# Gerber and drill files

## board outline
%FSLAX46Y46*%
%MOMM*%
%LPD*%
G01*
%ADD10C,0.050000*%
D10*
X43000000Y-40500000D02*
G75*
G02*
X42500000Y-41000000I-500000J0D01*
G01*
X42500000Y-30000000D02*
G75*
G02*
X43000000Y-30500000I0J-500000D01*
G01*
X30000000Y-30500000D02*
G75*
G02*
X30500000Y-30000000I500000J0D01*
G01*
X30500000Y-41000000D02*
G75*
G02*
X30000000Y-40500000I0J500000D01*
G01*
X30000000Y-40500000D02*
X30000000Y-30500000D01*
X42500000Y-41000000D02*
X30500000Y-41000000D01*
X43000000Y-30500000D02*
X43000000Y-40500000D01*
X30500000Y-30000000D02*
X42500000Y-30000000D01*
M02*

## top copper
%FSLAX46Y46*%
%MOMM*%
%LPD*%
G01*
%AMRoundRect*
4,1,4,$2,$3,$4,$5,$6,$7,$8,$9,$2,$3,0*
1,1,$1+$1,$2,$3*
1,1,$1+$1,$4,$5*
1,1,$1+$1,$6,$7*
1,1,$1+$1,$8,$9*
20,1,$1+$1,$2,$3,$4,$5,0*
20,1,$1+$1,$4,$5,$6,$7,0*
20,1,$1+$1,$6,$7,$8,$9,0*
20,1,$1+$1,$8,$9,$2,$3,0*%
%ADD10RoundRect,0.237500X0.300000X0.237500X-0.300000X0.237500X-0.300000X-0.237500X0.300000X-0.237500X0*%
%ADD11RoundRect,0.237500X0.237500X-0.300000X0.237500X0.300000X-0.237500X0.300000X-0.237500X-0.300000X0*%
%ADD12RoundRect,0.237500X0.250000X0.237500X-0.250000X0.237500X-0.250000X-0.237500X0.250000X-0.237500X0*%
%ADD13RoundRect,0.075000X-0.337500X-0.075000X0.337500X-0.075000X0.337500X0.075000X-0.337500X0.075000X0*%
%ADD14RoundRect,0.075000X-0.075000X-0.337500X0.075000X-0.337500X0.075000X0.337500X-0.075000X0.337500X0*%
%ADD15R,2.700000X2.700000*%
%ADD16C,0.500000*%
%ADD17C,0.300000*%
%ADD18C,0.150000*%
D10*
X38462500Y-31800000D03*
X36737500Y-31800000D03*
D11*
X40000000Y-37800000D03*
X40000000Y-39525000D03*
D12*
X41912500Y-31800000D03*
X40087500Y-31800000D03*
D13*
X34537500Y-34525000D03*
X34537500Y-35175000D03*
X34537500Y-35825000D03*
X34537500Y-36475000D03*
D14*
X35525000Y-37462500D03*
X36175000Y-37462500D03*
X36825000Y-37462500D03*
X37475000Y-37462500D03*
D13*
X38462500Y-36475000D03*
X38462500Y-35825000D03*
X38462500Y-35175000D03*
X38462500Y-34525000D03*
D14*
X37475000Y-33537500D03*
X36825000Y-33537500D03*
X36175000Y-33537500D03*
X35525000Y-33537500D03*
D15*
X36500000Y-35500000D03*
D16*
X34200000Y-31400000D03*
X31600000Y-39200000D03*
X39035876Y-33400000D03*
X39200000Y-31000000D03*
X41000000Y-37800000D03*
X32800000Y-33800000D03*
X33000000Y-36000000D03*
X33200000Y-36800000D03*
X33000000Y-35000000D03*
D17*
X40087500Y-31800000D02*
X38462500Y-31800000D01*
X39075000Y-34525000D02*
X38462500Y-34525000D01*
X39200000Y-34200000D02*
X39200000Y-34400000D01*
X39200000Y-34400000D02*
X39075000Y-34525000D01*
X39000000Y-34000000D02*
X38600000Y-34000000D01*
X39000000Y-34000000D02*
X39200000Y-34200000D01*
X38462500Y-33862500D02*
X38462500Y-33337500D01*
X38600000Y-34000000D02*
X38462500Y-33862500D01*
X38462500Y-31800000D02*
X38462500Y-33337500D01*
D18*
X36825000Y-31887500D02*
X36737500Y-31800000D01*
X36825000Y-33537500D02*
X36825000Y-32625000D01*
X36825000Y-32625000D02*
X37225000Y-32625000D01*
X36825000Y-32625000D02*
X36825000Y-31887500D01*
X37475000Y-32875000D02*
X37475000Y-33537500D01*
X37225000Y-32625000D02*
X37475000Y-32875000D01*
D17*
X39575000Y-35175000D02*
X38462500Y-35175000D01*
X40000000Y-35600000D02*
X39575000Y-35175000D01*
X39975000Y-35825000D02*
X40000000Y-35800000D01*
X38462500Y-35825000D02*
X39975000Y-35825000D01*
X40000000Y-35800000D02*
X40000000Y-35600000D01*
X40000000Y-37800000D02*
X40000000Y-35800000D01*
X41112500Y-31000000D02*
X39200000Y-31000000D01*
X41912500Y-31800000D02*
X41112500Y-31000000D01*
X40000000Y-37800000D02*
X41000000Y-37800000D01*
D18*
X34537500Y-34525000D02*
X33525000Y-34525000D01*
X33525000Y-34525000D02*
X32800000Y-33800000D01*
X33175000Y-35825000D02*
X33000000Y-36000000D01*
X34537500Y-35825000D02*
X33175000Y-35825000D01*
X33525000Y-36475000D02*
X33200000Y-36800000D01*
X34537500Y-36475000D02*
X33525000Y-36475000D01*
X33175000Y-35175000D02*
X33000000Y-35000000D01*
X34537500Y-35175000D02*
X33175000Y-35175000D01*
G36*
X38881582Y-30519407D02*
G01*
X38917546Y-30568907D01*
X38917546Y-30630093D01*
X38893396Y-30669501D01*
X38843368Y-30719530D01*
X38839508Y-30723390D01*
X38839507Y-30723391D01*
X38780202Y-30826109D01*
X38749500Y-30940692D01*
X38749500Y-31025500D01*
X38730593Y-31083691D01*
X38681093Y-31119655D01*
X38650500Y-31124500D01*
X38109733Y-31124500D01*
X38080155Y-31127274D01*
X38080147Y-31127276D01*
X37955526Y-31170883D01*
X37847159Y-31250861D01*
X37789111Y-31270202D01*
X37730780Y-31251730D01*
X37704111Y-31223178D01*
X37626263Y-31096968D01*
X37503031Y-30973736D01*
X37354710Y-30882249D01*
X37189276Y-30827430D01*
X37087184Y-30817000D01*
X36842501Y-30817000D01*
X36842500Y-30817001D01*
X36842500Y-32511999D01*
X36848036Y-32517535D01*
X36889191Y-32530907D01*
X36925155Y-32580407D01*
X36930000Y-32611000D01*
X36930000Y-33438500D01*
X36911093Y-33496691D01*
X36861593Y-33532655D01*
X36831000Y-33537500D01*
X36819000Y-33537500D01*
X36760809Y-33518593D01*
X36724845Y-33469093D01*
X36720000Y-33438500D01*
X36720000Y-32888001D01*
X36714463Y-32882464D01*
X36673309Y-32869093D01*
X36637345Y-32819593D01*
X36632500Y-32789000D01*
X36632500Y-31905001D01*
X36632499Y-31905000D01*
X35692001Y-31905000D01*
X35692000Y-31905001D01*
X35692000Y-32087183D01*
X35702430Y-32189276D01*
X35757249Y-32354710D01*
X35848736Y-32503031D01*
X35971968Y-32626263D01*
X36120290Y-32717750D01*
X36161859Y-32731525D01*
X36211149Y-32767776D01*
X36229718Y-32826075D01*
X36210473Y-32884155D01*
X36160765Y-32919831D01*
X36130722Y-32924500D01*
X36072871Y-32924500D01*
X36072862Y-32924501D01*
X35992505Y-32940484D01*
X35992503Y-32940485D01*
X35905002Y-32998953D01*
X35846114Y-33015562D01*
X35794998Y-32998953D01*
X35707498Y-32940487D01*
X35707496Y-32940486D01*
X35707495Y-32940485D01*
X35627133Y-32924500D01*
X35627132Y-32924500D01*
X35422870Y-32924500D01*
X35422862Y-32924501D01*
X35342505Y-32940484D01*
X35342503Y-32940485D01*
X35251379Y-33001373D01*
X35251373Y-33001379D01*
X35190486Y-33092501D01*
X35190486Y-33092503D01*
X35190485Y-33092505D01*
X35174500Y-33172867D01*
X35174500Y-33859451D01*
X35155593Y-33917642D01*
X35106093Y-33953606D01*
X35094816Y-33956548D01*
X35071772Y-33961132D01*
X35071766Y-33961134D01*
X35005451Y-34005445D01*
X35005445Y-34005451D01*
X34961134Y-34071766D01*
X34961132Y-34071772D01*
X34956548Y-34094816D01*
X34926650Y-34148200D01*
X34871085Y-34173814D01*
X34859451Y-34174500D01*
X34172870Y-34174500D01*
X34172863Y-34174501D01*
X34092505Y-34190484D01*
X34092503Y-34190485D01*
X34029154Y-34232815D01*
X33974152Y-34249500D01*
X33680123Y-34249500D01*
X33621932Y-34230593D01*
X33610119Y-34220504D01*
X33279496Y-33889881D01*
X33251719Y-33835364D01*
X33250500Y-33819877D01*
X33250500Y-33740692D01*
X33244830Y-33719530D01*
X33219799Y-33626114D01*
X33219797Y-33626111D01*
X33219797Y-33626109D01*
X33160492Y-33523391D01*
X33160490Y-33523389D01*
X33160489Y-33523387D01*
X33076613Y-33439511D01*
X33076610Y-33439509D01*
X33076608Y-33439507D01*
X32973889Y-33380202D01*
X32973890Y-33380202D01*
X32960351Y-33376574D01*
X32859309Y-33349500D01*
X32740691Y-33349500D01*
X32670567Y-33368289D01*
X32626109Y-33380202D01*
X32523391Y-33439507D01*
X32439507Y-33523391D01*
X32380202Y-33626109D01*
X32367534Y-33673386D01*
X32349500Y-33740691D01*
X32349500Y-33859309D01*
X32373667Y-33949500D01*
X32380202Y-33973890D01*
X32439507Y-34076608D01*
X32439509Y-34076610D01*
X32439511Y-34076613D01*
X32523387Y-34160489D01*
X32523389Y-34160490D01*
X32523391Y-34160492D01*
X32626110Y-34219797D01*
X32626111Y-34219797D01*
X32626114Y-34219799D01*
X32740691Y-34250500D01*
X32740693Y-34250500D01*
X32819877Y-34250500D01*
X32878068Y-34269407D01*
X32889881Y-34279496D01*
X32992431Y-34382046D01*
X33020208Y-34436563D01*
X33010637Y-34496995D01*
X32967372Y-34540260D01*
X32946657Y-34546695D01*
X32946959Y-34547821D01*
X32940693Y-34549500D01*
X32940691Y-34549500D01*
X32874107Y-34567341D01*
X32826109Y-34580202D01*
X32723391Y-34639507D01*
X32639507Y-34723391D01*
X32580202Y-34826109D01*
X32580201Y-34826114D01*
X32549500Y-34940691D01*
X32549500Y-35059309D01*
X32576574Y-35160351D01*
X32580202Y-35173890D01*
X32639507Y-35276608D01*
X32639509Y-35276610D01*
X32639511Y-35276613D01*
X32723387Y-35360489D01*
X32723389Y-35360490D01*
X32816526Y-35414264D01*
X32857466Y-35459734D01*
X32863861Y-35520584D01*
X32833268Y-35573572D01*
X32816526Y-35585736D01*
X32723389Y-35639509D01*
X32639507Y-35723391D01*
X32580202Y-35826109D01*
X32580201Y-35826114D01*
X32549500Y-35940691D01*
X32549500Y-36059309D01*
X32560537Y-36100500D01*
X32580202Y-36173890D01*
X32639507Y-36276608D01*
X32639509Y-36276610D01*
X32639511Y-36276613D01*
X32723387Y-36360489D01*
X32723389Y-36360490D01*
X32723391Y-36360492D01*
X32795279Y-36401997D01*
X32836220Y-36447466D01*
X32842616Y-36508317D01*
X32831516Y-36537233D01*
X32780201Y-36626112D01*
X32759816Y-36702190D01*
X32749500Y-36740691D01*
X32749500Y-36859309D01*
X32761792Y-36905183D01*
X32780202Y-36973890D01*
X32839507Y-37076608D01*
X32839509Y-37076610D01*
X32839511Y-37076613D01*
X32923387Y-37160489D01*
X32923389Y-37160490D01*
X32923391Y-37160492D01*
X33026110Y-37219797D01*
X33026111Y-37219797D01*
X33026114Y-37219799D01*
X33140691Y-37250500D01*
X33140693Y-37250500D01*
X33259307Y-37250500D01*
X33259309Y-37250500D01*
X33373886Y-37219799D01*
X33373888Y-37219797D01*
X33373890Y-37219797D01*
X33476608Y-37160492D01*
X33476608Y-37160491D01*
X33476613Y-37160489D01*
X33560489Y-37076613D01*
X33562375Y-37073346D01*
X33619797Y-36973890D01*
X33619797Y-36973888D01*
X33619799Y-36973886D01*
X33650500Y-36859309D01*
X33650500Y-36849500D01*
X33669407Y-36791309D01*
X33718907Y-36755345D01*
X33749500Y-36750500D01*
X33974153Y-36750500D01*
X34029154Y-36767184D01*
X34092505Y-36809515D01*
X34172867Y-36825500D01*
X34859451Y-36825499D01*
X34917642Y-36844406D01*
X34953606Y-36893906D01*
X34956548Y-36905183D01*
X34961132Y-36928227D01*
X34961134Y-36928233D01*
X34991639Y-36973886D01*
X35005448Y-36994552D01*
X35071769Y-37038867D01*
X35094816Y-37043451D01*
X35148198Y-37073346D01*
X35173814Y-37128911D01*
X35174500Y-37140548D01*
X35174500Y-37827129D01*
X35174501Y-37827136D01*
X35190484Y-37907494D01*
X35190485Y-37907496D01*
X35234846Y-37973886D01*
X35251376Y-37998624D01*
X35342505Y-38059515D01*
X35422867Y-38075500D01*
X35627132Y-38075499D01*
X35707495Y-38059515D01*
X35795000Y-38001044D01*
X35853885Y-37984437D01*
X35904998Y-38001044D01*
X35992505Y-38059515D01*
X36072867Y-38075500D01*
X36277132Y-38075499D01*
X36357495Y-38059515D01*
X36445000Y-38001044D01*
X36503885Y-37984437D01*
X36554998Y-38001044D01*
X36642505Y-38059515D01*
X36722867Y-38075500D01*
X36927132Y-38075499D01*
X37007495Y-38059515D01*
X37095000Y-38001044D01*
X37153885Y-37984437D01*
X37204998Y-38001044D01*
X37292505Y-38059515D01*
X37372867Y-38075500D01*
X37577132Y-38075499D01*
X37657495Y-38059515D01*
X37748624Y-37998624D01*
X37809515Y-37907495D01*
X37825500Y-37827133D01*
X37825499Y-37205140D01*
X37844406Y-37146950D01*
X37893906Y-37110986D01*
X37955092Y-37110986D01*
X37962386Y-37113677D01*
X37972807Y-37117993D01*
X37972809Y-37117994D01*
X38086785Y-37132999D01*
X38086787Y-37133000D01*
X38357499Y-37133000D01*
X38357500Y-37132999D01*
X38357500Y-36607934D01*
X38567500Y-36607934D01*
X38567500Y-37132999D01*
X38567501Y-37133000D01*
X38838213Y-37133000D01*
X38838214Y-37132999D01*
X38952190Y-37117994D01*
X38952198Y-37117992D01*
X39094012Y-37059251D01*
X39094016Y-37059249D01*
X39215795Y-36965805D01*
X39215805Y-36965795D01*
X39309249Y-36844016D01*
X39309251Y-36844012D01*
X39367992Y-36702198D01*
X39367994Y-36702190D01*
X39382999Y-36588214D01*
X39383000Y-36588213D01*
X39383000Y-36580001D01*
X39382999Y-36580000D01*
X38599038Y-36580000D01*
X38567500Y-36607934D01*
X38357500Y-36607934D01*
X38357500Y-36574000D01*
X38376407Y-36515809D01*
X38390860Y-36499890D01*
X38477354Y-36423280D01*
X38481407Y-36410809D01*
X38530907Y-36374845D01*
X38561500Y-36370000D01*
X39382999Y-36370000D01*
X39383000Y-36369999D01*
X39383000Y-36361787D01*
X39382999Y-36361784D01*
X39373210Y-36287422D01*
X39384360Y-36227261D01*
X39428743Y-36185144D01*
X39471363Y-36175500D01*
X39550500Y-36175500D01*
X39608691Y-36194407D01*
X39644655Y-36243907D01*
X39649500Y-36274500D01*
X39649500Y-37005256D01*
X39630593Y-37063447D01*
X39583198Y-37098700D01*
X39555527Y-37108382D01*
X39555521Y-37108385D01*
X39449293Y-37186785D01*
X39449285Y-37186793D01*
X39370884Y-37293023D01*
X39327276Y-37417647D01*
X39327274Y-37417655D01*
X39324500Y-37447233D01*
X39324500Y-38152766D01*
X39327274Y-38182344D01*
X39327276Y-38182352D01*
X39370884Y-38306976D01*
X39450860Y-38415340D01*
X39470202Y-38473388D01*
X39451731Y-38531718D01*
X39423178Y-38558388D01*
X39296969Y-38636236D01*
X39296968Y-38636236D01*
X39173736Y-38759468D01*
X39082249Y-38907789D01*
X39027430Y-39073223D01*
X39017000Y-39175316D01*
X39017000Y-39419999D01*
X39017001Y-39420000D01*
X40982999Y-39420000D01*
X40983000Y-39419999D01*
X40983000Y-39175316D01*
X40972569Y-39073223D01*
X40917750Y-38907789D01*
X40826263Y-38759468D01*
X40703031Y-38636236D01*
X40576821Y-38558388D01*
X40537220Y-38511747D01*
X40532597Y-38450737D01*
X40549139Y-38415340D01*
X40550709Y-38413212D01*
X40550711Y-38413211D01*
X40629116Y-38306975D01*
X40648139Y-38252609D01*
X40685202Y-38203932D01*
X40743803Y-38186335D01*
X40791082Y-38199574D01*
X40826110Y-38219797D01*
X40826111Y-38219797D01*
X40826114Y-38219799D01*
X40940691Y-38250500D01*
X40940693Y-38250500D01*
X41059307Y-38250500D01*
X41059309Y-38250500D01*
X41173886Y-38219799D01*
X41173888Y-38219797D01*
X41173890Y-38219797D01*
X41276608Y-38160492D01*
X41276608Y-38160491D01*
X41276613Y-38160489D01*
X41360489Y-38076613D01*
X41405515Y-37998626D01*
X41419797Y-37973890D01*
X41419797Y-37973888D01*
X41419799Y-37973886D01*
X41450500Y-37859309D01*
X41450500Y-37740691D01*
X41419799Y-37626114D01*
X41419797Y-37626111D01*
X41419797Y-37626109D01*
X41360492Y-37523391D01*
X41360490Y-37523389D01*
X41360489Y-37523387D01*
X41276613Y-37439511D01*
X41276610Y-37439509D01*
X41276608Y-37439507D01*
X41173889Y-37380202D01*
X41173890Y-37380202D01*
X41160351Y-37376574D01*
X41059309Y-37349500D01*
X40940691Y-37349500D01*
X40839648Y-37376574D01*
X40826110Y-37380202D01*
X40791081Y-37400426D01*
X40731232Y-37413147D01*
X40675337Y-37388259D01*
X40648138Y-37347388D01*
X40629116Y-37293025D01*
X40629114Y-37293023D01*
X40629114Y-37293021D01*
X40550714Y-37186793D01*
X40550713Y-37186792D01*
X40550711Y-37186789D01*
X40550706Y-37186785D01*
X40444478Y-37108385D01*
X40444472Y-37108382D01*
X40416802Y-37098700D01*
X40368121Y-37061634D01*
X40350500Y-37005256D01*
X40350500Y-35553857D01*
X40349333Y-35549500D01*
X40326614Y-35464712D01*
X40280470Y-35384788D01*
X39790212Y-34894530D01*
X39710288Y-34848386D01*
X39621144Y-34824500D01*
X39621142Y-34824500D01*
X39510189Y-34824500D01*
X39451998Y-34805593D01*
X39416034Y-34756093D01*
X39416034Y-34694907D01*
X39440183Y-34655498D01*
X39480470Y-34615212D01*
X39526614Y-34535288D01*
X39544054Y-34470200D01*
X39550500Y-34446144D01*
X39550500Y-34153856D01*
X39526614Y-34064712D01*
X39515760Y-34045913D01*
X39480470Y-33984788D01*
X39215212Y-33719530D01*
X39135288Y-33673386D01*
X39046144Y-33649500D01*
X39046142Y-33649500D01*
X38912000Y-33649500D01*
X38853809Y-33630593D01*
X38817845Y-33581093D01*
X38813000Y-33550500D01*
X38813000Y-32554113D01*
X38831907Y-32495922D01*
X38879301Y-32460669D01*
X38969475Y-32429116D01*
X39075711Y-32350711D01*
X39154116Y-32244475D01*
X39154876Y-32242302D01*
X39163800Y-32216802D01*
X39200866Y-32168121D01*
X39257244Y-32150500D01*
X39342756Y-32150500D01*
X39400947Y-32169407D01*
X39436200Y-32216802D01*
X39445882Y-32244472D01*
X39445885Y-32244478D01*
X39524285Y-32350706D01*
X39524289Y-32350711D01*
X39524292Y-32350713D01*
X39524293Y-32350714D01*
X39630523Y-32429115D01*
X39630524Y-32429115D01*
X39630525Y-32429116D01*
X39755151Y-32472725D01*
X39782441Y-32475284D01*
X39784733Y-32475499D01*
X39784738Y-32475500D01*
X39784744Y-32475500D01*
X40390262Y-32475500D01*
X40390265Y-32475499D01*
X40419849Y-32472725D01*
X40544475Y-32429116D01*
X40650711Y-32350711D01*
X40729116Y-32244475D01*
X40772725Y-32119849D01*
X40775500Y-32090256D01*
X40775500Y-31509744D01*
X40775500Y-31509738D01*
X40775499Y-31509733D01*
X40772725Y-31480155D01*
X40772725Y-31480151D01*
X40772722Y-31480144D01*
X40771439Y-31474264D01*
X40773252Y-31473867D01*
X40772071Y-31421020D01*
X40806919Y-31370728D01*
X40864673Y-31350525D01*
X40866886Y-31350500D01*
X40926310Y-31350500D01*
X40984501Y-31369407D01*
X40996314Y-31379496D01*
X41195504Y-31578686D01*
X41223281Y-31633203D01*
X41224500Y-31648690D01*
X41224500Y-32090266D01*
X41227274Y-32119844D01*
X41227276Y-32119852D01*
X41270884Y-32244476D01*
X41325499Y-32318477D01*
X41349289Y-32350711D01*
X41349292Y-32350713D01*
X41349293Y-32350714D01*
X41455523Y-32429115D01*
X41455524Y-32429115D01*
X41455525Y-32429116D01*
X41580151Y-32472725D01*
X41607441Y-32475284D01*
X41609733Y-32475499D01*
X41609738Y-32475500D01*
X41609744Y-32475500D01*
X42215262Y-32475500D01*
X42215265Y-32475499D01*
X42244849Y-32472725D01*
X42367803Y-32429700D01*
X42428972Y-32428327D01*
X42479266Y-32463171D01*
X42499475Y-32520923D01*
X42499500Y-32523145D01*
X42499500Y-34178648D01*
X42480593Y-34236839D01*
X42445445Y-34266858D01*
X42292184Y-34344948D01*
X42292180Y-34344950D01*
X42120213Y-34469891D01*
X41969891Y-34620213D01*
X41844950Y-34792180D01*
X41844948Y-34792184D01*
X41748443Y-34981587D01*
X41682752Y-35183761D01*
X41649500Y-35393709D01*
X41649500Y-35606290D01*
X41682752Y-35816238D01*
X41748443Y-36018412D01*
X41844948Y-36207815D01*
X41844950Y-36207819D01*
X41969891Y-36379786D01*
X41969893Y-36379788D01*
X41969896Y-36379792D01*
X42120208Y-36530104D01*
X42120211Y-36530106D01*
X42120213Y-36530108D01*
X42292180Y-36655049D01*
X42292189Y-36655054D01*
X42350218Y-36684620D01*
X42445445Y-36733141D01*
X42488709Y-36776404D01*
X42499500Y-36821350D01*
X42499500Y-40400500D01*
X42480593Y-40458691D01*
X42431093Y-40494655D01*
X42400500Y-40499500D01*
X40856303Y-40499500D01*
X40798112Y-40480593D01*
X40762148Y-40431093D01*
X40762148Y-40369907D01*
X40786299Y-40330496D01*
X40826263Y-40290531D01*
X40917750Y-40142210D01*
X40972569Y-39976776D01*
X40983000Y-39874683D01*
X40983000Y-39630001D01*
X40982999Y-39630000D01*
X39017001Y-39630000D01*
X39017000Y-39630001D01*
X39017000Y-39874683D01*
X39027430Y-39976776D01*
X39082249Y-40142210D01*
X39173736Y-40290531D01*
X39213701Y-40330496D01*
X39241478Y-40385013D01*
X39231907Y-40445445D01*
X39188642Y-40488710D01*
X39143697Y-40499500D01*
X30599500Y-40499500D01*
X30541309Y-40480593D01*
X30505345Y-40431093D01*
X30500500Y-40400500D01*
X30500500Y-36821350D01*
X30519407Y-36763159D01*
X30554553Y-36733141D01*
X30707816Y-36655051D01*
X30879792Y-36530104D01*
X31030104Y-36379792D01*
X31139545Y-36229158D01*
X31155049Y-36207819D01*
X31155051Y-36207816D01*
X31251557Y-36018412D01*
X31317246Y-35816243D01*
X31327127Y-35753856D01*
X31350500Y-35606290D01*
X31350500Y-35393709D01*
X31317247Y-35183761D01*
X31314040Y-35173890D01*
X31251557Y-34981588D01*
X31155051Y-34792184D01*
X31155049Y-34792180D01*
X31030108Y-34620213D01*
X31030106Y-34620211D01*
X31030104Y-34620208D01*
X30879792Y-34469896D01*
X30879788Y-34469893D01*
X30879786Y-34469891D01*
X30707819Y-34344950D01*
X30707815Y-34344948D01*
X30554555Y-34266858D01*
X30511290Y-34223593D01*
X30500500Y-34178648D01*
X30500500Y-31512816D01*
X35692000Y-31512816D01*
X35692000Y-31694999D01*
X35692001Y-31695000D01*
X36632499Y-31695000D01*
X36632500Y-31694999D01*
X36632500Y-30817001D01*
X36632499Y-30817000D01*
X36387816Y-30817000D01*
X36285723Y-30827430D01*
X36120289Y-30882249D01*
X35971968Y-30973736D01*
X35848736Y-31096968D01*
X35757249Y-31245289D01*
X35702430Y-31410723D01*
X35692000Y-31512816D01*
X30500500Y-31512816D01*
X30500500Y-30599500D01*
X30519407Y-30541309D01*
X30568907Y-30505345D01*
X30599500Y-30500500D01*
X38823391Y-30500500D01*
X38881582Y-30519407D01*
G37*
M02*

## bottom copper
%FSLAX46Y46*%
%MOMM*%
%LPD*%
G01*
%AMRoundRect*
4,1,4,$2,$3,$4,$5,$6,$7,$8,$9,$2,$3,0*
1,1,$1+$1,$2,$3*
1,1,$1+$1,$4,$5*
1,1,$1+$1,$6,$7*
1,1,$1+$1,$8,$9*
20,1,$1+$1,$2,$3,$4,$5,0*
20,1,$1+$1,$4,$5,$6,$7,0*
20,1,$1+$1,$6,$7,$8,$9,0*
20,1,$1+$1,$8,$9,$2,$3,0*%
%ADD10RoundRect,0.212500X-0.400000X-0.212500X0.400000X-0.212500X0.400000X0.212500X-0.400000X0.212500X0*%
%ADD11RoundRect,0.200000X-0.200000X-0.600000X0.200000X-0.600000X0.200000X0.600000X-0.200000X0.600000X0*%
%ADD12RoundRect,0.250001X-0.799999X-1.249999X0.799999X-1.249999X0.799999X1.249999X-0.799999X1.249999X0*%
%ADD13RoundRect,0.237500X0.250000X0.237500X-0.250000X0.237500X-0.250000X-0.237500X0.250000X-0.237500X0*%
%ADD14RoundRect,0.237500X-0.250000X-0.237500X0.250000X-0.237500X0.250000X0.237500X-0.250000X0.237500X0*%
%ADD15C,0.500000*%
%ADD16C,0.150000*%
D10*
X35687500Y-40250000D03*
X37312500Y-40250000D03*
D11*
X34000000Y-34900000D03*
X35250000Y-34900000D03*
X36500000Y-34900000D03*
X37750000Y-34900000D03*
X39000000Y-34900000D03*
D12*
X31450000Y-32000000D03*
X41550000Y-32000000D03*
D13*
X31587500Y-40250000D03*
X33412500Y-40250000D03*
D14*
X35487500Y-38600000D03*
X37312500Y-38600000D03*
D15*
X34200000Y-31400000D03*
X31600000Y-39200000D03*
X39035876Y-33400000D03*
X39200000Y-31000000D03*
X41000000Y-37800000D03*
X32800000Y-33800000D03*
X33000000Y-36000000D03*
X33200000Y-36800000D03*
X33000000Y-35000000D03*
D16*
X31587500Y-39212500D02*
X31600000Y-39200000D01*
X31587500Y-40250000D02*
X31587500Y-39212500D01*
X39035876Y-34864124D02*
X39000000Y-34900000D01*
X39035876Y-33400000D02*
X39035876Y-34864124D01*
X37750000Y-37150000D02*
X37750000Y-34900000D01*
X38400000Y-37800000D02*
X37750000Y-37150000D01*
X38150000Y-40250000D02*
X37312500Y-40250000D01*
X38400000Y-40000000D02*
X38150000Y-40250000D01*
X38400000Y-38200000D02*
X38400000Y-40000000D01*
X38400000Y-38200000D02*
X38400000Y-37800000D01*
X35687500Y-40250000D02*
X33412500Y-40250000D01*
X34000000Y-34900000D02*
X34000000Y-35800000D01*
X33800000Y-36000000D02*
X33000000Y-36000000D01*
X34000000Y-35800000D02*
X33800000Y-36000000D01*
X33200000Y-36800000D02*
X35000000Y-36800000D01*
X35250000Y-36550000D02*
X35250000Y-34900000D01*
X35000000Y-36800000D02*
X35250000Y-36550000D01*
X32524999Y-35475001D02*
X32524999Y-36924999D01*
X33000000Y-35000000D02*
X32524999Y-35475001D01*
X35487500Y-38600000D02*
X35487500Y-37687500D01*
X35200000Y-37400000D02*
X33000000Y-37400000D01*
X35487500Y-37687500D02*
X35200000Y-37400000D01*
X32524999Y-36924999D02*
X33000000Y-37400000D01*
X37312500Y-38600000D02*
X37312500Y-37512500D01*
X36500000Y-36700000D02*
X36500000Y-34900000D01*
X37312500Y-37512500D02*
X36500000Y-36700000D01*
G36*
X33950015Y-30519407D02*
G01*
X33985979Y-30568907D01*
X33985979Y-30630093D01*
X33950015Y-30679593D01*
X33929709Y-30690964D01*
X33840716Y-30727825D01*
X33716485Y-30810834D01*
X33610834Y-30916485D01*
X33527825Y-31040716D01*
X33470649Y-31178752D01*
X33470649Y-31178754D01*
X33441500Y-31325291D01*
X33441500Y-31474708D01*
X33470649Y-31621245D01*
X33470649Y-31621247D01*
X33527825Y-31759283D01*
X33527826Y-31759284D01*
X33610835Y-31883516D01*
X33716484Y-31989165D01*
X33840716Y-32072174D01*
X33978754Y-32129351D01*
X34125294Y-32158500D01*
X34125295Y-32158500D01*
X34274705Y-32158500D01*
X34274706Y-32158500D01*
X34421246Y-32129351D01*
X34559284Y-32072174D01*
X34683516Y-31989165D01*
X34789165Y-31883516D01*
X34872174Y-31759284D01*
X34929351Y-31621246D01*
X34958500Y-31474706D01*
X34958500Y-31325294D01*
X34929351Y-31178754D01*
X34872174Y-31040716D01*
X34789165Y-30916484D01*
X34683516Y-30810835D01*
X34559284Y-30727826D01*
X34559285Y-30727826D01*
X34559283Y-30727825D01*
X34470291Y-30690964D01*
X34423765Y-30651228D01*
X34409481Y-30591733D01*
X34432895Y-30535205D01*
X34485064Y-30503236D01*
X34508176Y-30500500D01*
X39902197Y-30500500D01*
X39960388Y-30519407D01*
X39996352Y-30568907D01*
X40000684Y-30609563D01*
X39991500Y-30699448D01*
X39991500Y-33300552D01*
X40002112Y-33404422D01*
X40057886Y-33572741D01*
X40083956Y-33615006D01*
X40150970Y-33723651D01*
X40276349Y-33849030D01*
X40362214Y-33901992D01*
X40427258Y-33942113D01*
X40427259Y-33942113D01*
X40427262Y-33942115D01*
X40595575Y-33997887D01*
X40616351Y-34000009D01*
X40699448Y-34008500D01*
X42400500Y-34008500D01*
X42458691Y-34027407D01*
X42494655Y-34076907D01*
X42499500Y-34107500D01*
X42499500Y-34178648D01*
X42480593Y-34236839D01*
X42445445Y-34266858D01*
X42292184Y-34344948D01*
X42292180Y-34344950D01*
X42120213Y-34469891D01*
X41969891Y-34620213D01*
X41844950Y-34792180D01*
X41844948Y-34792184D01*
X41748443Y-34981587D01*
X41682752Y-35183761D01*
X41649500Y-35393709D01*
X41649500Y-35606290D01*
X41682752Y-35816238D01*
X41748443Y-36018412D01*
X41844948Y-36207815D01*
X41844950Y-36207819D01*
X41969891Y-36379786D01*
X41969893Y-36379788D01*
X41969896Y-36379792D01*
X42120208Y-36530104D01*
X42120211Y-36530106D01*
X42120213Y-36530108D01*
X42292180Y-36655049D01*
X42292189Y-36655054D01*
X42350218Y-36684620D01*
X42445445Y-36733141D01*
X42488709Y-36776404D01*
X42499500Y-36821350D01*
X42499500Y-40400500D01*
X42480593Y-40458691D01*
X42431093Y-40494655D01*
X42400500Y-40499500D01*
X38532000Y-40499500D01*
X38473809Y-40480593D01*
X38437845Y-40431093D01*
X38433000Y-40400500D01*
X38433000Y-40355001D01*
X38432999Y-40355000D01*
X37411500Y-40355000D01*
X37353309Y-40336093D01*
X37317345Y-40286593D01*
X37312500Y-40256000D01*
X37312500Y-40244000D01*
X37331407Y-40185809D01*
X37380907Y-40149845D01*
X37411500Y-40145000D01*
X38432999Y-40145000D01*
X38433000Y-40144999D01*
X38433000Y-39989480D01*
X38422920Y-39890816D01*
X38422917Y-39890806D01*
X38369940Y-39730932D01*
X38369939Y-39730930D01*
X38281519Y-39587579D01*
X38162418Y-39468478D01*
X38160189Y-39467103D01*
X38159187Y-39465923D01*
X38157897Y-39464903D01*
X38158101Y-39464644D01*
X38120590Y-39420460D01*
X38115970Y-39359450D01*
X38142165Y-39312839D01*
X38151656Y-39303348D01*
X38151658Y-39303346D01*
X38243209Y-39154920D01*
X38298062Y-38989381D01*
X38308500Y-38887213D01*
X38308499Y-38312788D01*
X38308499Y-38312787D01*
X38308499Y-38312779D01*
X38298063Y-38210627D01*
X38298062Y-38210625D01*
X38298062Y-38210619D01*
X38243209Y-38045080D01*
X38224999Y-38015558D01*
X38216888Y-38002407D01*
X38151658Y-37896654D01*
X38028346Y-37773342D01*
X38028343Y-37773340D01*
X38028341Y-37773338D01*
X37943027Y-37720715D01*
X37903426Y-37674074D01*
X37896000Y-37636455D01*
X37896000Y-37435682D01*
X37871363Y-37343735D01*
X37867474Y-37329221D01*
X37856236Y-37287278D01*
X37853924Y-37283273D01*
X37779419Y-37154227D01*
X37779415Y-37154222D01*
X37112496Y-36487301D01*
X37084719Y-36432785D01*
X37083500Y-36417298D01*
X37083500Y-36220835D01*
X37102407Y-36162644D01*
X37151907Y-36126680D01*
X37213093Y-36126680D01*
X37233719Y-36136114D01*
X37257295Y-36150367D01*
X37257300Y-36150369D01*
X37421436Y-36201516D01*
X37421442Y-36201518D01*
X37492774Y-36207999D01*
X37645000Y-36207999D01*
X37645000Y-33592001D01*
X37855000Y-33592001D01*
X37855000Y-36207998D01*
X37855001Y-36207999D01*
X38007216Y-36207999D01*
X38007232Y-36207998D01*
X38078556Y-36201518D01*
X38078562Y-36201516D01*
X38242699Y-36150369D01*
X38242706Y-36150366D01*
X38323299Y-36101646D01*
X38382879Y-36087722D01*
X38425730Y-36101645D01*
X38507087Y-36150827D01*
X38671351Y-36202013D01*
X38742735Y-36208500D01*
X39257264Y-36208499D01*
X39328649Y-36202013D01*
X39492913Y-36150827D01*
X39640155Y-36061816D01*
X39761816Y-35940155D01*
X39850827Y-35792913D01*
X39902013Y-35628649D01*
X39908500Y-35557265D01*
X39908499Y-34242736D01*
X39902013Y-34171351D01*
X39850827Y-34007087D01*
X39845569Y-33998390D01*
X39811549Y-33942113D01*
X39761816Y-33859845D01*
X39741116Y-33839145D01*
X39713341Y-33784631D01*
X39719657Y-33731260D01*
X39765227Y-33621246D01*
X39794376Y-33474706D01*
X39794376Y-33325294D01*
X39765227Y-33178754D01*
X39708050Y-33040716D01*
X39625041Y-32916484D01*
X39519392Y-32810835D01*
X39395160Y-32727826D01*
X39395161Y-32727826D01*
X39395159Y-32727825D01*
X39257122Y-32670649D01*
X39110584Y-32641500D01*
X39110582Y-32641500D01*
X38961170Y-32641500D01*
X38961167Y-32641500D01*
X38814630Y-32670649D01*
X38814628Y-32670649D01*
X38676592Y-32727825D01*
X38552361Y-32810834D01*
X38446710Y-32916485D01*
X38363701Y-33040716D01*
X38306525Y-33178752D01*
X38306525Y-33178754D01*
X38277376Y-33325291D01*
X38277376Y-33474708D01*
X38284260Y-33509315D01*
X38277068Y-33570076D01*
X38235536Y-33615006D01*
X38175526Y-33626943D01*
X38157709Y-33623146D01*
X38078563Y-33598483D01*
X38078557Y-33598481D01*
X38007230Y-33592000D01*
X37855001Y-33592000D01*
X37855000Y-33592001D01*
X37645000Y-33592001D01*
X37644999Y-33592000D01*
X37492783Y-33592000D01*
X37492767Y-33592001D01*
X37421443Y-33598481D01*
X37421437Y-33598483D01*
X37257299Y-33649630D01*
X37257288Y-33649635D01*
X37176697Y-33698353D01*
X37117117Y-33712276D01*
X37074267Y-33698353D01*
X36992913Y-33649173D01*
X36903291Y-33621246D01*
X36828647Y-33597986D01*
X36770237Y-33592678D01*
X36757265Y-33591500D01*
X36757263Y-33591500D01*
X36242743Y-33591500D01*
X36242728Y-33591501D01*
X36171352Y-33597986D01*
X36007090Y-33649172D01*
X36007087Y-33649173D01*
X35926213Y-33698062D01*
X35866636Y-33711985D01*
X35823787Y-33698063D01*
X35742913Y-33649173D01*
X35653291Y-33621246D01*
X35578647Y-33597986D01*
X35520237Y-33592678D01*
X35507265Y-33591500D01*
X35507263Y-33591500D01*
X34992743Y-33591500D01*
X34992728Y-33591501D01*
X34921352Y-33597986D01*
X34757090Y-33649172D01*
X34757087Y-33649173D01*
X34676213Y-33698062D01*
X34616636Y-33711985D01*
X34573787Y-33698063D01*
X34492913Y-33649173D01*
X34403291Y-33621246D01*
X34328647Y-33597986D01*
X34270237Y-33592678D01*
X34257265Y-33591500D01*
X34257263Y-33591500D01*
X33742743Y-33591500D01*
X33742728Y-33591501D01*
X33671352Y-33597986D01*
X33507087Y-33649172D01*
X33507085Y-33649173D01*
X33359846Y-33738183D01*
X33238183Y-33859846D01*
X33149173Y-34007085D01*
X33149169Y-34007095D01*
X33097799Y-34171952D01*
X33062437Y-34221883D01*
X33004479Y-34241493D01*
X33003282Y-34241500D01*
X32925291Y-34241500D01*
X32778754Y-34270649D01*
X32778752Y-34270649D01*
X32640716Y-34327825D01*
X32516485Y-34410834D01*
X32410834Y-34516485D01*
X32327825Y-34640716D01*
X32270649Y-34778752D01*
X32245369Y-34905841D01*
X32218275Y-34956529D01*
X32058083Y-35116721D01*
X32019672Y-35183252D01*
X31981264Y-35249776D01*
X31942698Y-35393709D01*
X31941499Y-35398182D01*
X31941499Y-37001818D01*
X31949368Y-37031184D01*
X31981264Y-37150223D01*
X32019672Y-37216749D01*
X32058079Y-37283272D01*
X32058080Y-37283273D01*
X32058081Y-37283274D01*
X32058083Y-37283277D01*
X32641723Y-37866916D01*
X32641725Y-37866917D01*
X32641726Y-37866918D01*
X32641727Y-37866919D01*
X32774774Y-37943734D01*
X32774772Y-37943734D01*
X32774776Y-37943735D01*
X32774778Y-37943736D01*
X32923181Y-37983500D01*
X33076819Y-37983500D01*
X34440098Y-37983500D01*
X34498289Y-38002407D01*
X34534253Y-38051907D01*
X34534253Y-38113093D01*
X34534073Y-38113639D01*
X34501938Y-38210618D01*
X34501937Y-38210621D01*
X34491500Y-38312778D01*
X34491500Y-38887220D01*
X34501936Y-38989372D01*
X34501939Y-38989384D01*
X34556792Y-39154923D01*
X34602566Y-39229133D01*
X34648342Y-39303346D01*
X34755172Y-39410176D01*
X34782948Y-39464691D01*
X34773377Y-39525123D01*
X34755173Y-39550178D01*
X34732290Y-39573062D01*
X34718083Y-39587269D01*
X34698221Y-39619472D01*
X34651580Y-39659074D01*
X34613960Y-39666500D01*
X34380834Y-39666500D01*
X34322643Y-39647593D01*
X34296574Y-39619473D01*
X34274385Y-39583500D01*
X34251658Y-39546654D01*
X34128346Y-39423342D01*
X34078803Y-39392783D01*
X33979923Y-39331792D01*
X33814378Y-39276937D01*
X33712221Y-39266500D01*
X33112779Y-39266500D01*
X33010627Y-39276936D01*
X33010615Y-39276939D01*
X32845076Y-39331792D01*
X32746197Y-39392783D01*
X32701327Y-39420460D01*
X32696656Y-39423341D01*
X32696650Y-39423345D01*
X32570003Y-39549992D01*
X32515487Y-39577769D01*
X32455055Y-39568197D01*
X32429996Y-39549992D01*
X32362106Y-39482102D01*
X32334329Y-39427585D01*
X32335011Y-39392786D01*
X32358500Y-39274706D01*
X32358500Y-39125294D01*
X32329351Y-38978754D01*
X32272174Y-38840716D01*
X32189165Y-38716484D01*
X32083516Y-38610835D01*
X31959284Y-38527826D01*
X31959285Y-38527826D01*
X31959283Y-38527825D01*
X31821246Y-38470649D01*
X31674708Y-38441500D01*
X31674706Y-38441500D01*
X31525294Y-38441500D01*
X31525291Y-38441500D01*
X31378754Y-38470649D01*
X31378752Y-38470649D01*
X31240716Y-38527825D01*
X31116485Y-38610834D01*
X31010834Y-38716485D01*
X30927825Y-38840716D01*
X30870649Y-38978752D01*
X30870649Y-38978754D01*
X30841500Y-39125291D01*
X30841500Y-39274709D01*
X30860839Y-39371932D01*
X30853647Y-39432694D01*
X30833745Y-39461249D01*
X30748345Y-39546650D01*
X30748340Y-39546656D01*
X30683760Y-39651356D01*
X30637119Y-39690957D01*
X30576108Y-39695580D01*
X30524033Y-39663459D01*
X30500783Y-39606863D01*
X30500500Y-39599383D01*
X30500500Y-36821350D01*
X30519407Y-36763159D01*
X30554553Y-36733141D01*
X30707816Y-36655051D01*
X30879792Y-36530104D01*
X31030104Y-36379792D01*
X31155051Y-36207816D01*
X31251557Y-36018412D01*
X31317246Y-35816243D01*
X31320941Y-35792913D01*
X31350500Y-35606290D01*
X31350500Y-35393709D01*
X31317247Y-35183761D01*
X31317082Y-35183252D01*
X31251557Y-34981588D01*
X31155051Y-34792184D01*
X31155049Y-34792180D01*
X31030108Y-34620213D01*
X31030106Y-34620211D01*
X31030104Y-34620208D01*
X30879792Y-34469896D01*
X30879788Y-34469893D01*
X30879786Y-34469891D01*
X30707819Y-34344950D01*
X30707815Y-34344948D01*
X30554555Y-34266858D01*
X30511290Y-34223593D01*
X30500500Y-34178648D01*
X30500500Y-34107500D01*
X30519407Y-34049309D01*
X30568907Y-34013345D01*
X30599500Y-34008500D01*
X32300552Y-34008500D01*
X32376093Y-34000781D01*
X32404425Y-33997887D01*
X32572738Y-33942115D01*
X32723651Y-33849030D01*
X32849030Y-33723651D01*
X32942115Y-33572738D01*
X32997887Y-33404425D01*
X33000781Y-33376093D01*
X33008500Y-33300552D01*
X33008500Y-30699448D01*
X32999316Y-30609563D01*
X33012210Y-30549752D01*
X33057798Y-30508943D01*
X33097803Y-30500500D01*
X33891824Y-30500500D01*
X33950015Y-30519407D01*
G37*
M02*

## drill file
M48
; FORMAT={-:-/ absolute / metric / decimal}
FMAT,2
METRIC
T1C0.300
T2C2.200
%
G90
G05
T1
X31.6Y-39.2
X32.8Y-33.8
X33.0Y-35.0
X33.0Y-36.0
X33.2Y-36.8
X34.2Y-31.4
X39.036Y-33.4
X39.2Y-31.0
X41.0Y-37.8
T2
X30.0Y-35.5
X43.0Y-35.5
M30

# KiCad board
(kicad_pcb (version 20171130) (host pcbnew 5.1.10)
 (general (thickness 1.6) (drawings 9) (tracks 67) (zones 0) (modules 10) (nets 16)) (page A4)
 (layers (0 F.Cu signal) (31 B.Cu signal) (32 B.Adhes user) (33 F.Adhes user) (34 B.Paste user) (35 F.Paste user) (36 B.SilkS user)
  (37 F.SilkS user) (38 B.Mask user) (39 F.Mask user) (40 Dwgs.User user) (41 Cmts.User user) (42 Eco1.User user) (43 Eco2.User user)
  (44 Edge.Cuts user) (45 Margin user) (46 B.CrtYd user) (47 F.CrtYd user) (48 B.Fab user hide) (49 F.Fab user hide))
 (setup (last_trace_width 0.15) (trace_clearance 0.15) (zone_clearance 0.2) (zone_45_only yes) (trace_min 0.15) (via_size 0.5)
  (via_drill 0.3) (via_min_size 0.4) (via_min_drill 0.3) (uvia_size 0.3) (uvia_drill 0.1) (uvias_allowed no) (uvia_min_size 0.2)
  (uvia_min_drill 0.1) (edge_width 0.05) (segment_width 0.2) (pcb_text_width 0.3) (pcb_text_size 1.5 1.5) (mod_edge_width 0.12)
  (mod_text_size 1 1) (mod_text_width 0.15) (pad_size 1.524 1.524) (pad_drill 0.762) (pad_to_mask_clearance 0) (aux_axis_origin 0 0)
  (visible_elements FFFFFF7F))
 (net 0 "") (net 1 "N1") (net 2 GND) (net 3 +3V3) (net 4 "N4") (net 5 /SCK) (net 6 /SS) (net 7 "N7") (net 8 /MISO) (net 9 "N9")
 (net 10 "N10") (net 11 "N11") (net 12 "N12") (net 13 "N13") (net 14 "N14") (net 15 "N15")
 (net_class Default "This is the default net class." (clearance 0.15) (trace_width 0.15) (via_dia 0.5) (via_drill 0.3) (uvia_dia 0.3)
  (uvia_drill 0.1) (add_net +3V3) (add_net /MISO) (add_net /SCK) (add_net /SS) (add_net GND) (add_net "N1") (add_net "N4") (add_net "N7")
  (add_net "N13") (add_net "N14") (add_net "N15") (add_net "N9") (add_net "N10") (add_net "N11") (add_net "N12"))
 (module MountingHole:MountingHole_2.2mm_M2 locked (layer F.Cu) (at 43 35.5)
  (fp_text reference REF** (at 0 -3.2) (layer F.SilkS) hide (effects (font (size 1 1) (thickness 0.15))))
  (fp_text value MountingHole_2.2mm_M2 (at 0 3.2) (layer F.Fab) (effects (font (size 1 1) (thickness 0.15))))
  (pad 1 np_thru_hole circle (at 0 0) (size 2.2 2.2) (drill 2.2) (layers *.Cu *.Mask)))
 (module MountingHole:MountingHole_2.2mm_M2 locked (layer F.Cu) (at 30 35.5)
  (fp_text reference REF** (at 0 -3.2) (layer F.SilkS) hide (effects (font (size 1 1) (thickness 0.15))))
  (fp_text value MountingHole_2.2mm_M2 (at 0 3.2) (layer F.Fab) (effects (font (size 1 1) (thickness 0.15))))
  (pad 1 np_thru_hole circle (at 0 0) (size 2.2 2.2) (drill 2.2) (layers *.Cu *.Mask)))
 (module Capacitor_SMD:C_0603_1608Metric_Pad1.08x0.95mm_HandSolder (layer F.Cu) (at 37.6 31.8 180)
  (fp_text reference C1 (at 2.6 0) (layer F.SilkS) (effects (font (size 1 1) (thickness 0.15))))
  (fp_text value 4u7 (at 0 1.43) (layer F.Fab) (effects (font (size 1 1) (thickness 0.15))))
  (pad 1 smd roundrect (at -0.8625 0 180) (size 1.075 0.95) (layers F.Cu F.Paste F.Mask) (roundrect_rratio 0.25) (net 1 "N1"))
  (pad 2 smd roundrect (at 0.8625 0 180) (size 1.075 0.95) (layers F.Cu F.Paste F.Mask) (roundrect_rratio 0.25) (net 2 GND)))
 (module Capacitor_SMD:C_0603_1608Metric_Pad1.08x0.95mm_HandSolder (layer F.Cu) (at 40 38.6625 90)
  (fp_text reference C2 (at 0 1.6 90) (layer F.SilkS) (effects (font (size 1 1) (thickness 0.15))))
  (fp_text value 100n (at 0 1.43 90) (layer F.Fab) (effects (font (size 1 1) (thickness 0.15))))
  (pad 2 smd roundrect (at 0.8625 0 90) (size 1.075 0.95) (layers F.Cu F.Paste F.Mask) (roundrect_rratio 0.25) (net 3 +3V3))
  (pad 1 smd roundrect (at -0.8625 0 90) (size 1.075 0.95) (layers F.Cu F.Paste F.Mask) (roundrect_rratio 0.25) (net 2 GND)))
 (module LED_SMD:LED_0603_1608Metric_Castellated (layer B.Cu) (at 36.5 40.25)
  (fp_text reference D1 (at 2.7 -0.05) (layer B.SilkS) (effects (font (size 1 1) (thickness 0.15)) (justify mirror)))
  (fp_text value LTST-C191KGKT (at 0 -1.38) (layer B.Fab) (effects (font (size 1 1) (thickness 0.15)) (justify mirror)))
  (pad 1 smd roundrect (at -0.8125 0) (size 1.225 0.85) (layers B.Cu B.Paste B.Mask) (roundrect_rratio 0.25) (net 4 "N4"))
  (pad 2 smd roundrect (at 0.8125 0) (size 1.225 0.85) (layers B.Cu B.Paste B.Mask) (roundrect_rratio 0.25) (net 3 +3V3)))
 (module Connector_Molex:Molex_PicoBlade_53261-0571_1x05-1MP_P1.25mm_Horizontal (layer B.Cu) (at 36.5 32.5)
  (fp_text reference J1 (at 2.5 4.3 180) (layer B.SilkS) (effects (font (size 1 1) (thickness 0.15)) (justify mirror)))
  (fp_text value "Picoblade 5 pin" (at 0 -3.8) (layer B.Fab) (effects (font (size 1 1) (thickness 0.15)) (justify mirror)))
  (pad 1 smd roundrect (at -2.5 2.4) (size 0.8 1.6) (layers B.Cu B.Paste B.Mask) (roundrect_rratio 0.25) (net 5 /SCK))
  (pad 2 smd roundrect (at -1.25 2.4) (size 0.8 1.6) (layers B.Cu B.Paste B.Mask) (roundrect_rratio 0.25) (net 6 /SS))
  (pad 3 smd roundrect (at 0 2.4) (size 0.8 1.6) (layers B.Cu B.Paste B.Mask) (roundrect_rratio 0.25) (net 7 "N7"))
  (pad 4 smd roundrect (at 1.25 2.4) (size 0.8 1.6) (layers B.Cu B.Paste B.Mask) (roundrect_rratio 0.25) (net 3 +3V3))
  (pad 5 smd roundrect (at 2.5 2.4) (size 0.8 1.6) (layers B.Cu B.Paste B.Mask) (roundrect_rratio 0.25) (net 2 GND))
  (pad MP smd roundrect (at -5.05 -0.5) (size 2.1 3) (layers B.Cu B.Paste B.Mask) (roundrect_rratio 0.119048))
  (pad MP smd roundrect (at 5.05 -0.5) (size 2.1 3) (layers B.Cu B.Paste B.Mask) (roundrect_rratio 0.119048)))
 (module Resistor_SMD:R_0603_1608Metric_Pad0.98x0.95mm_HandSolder (layer F.Cu) (at 41 31.8 180)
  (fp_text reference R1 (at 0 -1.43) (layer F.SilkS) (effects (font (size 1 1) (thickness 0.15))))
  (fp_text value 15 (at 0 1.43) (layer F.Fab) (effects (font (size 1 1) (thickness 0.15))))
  (pad 1 smd roundrect (at -0.9125 0 180) (size 0.975 0.95) (layers F.Cu F.Paste F.Mask) (roundrect_rratio 0.25) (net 3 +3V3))
  (pad 2 smd roundrect (at 0.9125 0 180) (size 0.975 0.95) (layers F.Cu F.Paste F.Mask) (roundrect_rratio 0.25) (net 1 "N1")))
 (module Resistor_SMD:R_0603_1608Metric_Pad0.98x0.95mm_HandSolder (layer B.Cu) (at 32.5 40.25 180)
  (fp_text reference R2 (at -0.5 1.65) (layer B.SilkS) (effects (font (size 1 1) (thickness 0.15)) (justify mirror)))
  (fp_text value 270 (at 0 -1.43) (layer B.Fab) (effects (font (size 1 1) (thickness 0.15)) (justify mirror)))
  (pad 2 smd roundrect (at 0.9125 0 180) (size 0.975 0.95) (layers B.Cu B.Paste B.Mask) (roundrect_rratio 0.25) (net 2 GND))
  (pad 1 smd roundrect (at -0.9125 0 180) (size 0.975 0.95) (layers B.Cu B.Paste B.Mask) (roundrect_rratio 0.25) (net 4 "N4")))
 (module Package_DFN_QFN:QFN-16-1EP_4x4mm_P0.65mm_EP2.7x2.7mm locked (layer F.Cu) (at 36.5 35.5)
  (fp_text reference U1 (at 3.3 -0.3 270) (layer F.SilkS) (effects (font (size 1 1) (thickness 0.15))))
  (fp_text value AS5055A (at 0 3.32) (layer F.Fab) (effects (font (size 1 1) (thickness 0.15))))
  (pad 1 smd roundrect (at -1.9625 -0.975) (size 0.825 0.3) (layers F.Cu F.Paste F.Mask) (roundrect_rratio 0.25) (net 3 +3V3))
  (pad 2 smd roundrect (at -1.9625 -0.325) (size 0.825 0.3) (layers F.Cu F.Paste F.Mask) (roundrect_rratio 0.25) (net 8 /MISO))
  (pad 3 smd roundrect (at -1.9625 0.325) (size 0.825 0.3) (layers F.Cu F.Paste F.Mask) (roundrect_rratio 0.25) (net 5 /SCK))
  (pad 4 smd roundrect (at -1.9625 0.975) (size 0.825 0.3) (layers F.Cu F.Paste F.Mask) (roundrect_rratio 0.25) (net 6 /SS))
  (pad 5 smd roundrect (at -0.975 1.9625) (size 0.3 0.825) (layers F.Cu F.Paste F.Mask) (roundrect_rratio 0.25) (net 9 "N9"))
  (pad 6 smd roundrect (at -0.325 1.9625) (size 0.3 0.825) (layers F.Cu F.Paste F.Mask) (roundrect_rratio 0.25) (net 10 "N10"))
  (pad 7 smd roundrect (at 0.325 1.9625) (size 0.3 0.825) (layers F.Cu F.Paste F.Mask) (roundrect_rratio 0.25) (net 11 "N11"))
  (pad 8 smd roundrect (at 0.975 1.9625) (size 0.3 0.825) (layers F.Cu F.Paste F.Mask) (roundrect_rratio 0.25) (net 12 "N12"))
  (pad 9 smd roundrect (at 1.9625 0.975) (size 0.825 0.3) (layers F.Cu F.Paste F.Mask) (roundrect_rratio 0.25) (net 2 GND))
  (pad 10 smd roundrect (at 1.9625 0.325) (size 0.825 0.3) (layers F.Cu F.Paste F.Mask) (roundrect_rratio 0.25) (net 3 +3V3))
  (pad 11 smd roundrect (at 1.9625 -0.325) (size 0.825 0.3) (layers F.Cu F.Paste F.Mask) (roundrect_rratio 0.25) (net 3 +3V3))
  (pad 12 smd roundrect (at 1.9625 -0.975) (size 0.825 0.3) (layers F.Cu F.Paste F.Mask) (roundrect_rratio 0.25) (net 1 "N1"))
  (pad 13 smd roundrect (at 0.975 -1.9625) (size 0.3 0.825) (layers F.Cu F.Paste F.Mask) (roundrect_rratio 0.25) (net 2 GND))
  (pad 14 smd roundrect (at 0.325 -1.9625) (size 0.3 0.825) (layers F.Cu F.Paste F.Mask) (roundrect_rratio 0.25) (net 2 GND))
  (pad 15 smd roundrect (at -0.325 -1.9625) (size 0.3 0.825) (layers F.Cu F.Paste F.Mask) (roundrect_rratio 0.25) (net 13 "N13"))
  (pad 16 smd roundrect (at -0.975 -1.9625) (size 0.3 0.825) (layers F.Cu F.Paste F.Mask) (roundrect_rratio 0.25) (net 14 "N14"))
  (pad 17 smd rect (at 0 0) (size 2.7 2.7) (layers F.Cu F.Mask) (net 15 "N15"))
  (pad "" smd roundrect (at -0.675 -0.675) (size 1.09 1.09) (layers F.Paste) (roundrect_rratio 0.229358))
  (pad "" smd roundrect (at -0.675 0.675) (size 1.09 1.09) (layers F.Paste) (roundrect_rratio 0.229358))
  (pad "" smd roundrect (at 0.675 -0.675) (size 1.09 1.09) (layers F.Paste) (roundrect_rratio 0.229358))
  (pad "" smd roundrect (at 0.675 0.675) (size 1.09 1.09) (layers F.Paste) (roundrect_rratio 0.229358)))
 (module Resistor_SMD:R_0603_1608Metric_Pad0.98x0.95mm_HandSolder (layer B.Cu) (at 36.4 38.6)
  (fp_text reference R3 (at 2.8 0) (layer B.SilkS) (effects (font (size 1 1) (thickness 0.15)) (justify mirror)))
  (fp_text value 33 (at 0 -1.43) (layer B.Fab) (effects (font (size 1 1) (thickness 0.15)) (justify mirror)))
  (pad 1 smd roundrect (at -0.9125 0) (size 0.975 0.95) (layers B.Cu B.Paste B.Mask) (roundrect_rratio 0.25) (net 8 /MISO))
  (pad 2 smd roundrect (at 0.9125 0) (size 0.975 0.95) (layers B.Cu B.Paste B.Mask) (roundrect_rratio 0.25) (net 7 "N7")))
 (gr_arc (start 42.5 40.5) (end 42.5 41) (angle -90) (layer Edge.Cuts) (width 0.05))
 (gr_arc (start 42.5 30.5) (end 43 30.5) (angle -90) (layer Edge.Cuts) (width 0.05))
 (gr_arc (start 30.5 30.5) (end 30.5 30) (angle -90) (layer Edge.Cuts) (width 0.05))
 (gr_arc (start 30.5 40.5) (end 30 40.5) (angle -90) (layer Edge.Cuts) (width 0.05))
 (gr_line (start 30 40.5) (end 30 30.5) (layer Edge.Cuts) (width 0.05))
 (gr_line (start 42.5 41) (end 30.5 41) (layer Edge.Cuts) (width 0.05))
 (gr_line (start 43 30.5) (end 43 40.5) (layer Edge.Cuts) (width 0.05))
 (gr_line (start 30.5 30) (end 42.5 30) (layer Edge.Cuts) (width 0.05))
 (via (at 34.2 31.4) (size 0.5) (drill 0.3) (layers F.Cu B.Cu) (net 2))
 (segment (start 40.0875 31.8) (end 38.4625 31.8) (width 0.3) (layer F.Cu) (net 1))
 (segment (start 39.075 34.525) (end 38.4625 34.525) (width 0.3) (layer F.Cu) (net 1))
 (segment (start 39.2 34.2) (end 39.2 34.4) (width 0.3) (layer F.Cu) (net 1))
 (segment (start 39.2 34.4) (end 39.075 34.525) (width 0.3) (layer F.Cu) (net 1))
 (segment (start 39 34) (end 38.6 34) (width 0.3) (layer F.Cu) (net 1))
 (segment (start 39 34) (end 39.2 34.2) (width 0.3) (layer F.Cu) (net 1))
 (segment (start 38.4625 33.8625) (end 38.4625 33.3375) (width 0.3) (layer F.Cu) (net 1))
 (segment (start 38.6 34) (end 38.4625 33.8625) (width 0.3) (layer F.Cu) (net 1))
 (segment (start 38.4625 31.8) (end 38.4625 33.3375) (width 0.3) (layer F.Cu) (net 1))
 (segment (start 36.825 31.8875) (end 36.7375 31.8) (width 0.15) (layer F.Cu) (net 2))
 (segment (start 36.825 33.5375) (end 36.825 32.625) (width 0.15) (layer F.Cu) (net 2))
 (segment (start 36.825 32.625) (end 37.225 32.625) (width 0.15) (layer F.Cu) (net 2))
 (segment (start 36.825 32.625) (end 36.825 31.8875) (width 0.15) (layer F.Cu) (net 2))
 (segment (start 37.475 32.875) (end 37.475 33.5375) (width 0.15) (layer F.Cu) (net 2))
 (segment (start 37.225 32.625) (end 37.475 32.875) (width 0.15) (layer F.Cu) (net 2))
 (via (at 31.6 39.2) (size 0.5) (drill 0.3) (layers F.Cu B.Cu) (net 2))
 (segment (start 31.5875 39.2125) (end 31.6 39.2) (width 0.15) (layer B.Cu) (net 2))
 (segment (start 31.5875 40.25) (end 31.5875 39.2125) (width 0.15) (layer B.Cu) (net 2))
 (via (at 39.035876 33.4) (size 0.5) (drill 0.3) (layers F.Cu B.Cu) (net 2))
 (segment (start 39.035876 34.864124) (end 39 34.9) (width 0.15) (layer B.Cu) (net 2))
 (segment (start 39.035876 33.4) (end 39.035876 34.864124) (width 0.15) (layer B.Cu) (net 2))
 (segment (start 39.575 35.175) (end 38.4625 35.175) (width 0.3) (layer F.Cu) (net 3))
 (segment (start 40 35.6) (end 39.575 35.175) (width 0.3) (layer F.Cu) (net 3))
 (segment (start 39.975 35.825) (end 40 35.8) (width 0.3) (layer F.Cu) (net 3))
 (segment (start 38.4625 35.825) (end 39.975 35.825) (width 0.3) (layer F.Cu) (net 3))
 (segment (start 40 35.8) (end 40 35.6) (width 0.3) (layer F.Cu) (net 3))
 (segment (start 40 37.8) (end 40 35.8) (width 0.3) (layer F.Cu) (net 3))
 (via (at 39.2 31) (size 0.5) (drill 0.3) (layers F.Cu B.Cu) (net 3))
 (segment (start 41.1125 31) (end 39.2 31) (width 0.3) (layer F.Cu) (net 3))
 (segment (start 41.9125 31.8) (end 41.1125 31) (width 0.3) (layer F.Cu) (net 3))
 (segment (start 37.75 37.15) (end 37.75 34.9) (width 0.15) (layer B.Cu) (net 3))
 (segment (start 38.4 37.8) (end 37.75 37.15) (width 0.15) (layer B.Cu) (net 3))
 (segment (start 38.15 40.25) (end 37.3125 40.25) (width 0.15) (layer B.Cu) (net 3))
 (segment (start 38.4 40) (end 38.15 40.25) (width 0.15) (layer B.Cu) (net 3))
 (segment (start 38.4 38.2) (end 38.4 40) (width 0.15) (layer B.Cu) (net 3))
 (segment (start 38.4 38.2) (end 38.4 37.8) (width 0.15) (layer B.Cu) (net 3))
 (via (at 41 37.8) (size 0.5) (drill 0.3) (layers F.Cu B.Cu) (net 3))
 (segment (start 40 37.8) (end 41 37.8) (width 0.3) (layer F.Cu) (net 3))
 (segment (start 34.5375 34.525) (end 33.525 34.525) (width 0.15) (layer F.Cu) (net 3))
 (via (at 32.8 33.8) (size 0.5) (drill 0.3) (layers F.Cu B.Cu) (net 3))
 (segment (start 33.525 34.525) (end 32.8 33.8) (width 0.15) (layer F.Cu) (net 3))
 (segment (start 35.6875 40.25) (end 33.4125 40.25) (width 0.15) (layer B.Cu) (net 4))
 (segment (start 34 34.9) (end 34 35.8) (width 0.15) (layer B.Cu) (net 5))
 (via (at 33 36) (size 0.5) (drill 0.3) (layers F.Cu B.Cu) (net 5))
 (segment (start 33.8 36) (end 33 36) (width 0.15) (layer B.Cu) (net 5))
 (segment (start 34 35.8) (end 33.8 36) (width 0.15) (layer B.Cu) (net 5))
 (segment (start 33.175 35.825) (end 33 36) (width 0.15) (layer F.Cu) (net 5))
 (segment (start 34.5375 35.825) (end 33.175 35.825) (width 0.15) (layer F.Cu) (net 5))
 (via (at 33.2 36.8) (size 0.5) (drill 0.3) (layers F.Cu B.Cu) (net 6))
 (segment (start 33.525 36.475) (end 33.2 36.8) (width 0.15) (layer F.Cu) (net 6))
 (segment (start 34.5375 36.475) (end 33.525 36.475) (width 0.15) (layer F.Cu) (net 6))
 (segment (start 33.2 36.8) (end 35 36.8) (width 0.15) (layer B.Cu) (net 6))
 (segment (start 35.25 36.55) (end 35.25 34.9) (width 0.15) (layer B.Cu) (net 6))
 (segment (start 35 36.8) (end 35.25 36.55) (width 0.15) (layer B.Cu) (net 6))
 (via (at 33 35) (size 0.5) (drill 0.3) (layers F.Cu B.Cu) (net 8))
 (segment (start 33.175 35.175) (end 33 35) (width 0.15) (layer F.Cu) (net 8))
 (segment (start 34.5375 35.175) (end 33.175 35.175) (width 0.15) (layer F.Cu) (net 8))
 (segment (start 32.524999 35.475001) (end 32.524999 36.924999) (width 0.15) (layer B.Cu) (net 8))
 (segment (start 33 35) (end 32.524999 35.475001) (width 0.15) (layer B.Cu) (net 8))
 (segment (start 35.4875 38.6) (end 35.4875 37.6875) (width 0.15) (layer B.Cu) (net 8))
 (segment (start 35.2 37.4) (end 33 37.4) (width 0.15) (layer B.Cu) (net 8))
 (segment (start 35.4875 37.6875) (end 35.2 37.4) (width 0.15) (layer B.Cu) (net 8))
 (segment (start 32.524999 36.924999) (end 33 37.4) (width 0.15) (layer B.Cu) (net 8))
 (segment (start 37.3125 38.6) (end 37.3125 37.5125) (width 0.15) (layer B.Cu) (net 7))
 (segment (start 36.5 36.7) (end 36.5 34.9) (width 0.15) (layer B.Cu) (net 7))
 (segment (start 37.3125 37.5125) (end 36.5 36.7) (width 0.15) (layer B.Cu) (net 7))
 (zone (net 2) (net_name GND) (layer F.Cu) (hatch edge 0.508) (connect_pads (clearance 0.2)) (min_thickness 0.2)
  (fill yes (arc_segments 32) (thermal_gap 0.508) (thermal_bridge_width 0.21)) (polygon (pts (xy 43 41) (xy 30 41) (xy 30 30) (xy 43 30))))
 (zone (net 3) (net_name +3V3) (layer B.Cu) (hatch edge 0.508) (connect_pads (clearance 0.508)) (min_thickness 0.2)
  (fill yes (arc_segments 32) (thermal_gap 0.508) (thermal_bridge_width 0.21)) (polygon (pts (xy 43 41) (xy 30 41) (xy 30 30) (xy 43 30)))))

